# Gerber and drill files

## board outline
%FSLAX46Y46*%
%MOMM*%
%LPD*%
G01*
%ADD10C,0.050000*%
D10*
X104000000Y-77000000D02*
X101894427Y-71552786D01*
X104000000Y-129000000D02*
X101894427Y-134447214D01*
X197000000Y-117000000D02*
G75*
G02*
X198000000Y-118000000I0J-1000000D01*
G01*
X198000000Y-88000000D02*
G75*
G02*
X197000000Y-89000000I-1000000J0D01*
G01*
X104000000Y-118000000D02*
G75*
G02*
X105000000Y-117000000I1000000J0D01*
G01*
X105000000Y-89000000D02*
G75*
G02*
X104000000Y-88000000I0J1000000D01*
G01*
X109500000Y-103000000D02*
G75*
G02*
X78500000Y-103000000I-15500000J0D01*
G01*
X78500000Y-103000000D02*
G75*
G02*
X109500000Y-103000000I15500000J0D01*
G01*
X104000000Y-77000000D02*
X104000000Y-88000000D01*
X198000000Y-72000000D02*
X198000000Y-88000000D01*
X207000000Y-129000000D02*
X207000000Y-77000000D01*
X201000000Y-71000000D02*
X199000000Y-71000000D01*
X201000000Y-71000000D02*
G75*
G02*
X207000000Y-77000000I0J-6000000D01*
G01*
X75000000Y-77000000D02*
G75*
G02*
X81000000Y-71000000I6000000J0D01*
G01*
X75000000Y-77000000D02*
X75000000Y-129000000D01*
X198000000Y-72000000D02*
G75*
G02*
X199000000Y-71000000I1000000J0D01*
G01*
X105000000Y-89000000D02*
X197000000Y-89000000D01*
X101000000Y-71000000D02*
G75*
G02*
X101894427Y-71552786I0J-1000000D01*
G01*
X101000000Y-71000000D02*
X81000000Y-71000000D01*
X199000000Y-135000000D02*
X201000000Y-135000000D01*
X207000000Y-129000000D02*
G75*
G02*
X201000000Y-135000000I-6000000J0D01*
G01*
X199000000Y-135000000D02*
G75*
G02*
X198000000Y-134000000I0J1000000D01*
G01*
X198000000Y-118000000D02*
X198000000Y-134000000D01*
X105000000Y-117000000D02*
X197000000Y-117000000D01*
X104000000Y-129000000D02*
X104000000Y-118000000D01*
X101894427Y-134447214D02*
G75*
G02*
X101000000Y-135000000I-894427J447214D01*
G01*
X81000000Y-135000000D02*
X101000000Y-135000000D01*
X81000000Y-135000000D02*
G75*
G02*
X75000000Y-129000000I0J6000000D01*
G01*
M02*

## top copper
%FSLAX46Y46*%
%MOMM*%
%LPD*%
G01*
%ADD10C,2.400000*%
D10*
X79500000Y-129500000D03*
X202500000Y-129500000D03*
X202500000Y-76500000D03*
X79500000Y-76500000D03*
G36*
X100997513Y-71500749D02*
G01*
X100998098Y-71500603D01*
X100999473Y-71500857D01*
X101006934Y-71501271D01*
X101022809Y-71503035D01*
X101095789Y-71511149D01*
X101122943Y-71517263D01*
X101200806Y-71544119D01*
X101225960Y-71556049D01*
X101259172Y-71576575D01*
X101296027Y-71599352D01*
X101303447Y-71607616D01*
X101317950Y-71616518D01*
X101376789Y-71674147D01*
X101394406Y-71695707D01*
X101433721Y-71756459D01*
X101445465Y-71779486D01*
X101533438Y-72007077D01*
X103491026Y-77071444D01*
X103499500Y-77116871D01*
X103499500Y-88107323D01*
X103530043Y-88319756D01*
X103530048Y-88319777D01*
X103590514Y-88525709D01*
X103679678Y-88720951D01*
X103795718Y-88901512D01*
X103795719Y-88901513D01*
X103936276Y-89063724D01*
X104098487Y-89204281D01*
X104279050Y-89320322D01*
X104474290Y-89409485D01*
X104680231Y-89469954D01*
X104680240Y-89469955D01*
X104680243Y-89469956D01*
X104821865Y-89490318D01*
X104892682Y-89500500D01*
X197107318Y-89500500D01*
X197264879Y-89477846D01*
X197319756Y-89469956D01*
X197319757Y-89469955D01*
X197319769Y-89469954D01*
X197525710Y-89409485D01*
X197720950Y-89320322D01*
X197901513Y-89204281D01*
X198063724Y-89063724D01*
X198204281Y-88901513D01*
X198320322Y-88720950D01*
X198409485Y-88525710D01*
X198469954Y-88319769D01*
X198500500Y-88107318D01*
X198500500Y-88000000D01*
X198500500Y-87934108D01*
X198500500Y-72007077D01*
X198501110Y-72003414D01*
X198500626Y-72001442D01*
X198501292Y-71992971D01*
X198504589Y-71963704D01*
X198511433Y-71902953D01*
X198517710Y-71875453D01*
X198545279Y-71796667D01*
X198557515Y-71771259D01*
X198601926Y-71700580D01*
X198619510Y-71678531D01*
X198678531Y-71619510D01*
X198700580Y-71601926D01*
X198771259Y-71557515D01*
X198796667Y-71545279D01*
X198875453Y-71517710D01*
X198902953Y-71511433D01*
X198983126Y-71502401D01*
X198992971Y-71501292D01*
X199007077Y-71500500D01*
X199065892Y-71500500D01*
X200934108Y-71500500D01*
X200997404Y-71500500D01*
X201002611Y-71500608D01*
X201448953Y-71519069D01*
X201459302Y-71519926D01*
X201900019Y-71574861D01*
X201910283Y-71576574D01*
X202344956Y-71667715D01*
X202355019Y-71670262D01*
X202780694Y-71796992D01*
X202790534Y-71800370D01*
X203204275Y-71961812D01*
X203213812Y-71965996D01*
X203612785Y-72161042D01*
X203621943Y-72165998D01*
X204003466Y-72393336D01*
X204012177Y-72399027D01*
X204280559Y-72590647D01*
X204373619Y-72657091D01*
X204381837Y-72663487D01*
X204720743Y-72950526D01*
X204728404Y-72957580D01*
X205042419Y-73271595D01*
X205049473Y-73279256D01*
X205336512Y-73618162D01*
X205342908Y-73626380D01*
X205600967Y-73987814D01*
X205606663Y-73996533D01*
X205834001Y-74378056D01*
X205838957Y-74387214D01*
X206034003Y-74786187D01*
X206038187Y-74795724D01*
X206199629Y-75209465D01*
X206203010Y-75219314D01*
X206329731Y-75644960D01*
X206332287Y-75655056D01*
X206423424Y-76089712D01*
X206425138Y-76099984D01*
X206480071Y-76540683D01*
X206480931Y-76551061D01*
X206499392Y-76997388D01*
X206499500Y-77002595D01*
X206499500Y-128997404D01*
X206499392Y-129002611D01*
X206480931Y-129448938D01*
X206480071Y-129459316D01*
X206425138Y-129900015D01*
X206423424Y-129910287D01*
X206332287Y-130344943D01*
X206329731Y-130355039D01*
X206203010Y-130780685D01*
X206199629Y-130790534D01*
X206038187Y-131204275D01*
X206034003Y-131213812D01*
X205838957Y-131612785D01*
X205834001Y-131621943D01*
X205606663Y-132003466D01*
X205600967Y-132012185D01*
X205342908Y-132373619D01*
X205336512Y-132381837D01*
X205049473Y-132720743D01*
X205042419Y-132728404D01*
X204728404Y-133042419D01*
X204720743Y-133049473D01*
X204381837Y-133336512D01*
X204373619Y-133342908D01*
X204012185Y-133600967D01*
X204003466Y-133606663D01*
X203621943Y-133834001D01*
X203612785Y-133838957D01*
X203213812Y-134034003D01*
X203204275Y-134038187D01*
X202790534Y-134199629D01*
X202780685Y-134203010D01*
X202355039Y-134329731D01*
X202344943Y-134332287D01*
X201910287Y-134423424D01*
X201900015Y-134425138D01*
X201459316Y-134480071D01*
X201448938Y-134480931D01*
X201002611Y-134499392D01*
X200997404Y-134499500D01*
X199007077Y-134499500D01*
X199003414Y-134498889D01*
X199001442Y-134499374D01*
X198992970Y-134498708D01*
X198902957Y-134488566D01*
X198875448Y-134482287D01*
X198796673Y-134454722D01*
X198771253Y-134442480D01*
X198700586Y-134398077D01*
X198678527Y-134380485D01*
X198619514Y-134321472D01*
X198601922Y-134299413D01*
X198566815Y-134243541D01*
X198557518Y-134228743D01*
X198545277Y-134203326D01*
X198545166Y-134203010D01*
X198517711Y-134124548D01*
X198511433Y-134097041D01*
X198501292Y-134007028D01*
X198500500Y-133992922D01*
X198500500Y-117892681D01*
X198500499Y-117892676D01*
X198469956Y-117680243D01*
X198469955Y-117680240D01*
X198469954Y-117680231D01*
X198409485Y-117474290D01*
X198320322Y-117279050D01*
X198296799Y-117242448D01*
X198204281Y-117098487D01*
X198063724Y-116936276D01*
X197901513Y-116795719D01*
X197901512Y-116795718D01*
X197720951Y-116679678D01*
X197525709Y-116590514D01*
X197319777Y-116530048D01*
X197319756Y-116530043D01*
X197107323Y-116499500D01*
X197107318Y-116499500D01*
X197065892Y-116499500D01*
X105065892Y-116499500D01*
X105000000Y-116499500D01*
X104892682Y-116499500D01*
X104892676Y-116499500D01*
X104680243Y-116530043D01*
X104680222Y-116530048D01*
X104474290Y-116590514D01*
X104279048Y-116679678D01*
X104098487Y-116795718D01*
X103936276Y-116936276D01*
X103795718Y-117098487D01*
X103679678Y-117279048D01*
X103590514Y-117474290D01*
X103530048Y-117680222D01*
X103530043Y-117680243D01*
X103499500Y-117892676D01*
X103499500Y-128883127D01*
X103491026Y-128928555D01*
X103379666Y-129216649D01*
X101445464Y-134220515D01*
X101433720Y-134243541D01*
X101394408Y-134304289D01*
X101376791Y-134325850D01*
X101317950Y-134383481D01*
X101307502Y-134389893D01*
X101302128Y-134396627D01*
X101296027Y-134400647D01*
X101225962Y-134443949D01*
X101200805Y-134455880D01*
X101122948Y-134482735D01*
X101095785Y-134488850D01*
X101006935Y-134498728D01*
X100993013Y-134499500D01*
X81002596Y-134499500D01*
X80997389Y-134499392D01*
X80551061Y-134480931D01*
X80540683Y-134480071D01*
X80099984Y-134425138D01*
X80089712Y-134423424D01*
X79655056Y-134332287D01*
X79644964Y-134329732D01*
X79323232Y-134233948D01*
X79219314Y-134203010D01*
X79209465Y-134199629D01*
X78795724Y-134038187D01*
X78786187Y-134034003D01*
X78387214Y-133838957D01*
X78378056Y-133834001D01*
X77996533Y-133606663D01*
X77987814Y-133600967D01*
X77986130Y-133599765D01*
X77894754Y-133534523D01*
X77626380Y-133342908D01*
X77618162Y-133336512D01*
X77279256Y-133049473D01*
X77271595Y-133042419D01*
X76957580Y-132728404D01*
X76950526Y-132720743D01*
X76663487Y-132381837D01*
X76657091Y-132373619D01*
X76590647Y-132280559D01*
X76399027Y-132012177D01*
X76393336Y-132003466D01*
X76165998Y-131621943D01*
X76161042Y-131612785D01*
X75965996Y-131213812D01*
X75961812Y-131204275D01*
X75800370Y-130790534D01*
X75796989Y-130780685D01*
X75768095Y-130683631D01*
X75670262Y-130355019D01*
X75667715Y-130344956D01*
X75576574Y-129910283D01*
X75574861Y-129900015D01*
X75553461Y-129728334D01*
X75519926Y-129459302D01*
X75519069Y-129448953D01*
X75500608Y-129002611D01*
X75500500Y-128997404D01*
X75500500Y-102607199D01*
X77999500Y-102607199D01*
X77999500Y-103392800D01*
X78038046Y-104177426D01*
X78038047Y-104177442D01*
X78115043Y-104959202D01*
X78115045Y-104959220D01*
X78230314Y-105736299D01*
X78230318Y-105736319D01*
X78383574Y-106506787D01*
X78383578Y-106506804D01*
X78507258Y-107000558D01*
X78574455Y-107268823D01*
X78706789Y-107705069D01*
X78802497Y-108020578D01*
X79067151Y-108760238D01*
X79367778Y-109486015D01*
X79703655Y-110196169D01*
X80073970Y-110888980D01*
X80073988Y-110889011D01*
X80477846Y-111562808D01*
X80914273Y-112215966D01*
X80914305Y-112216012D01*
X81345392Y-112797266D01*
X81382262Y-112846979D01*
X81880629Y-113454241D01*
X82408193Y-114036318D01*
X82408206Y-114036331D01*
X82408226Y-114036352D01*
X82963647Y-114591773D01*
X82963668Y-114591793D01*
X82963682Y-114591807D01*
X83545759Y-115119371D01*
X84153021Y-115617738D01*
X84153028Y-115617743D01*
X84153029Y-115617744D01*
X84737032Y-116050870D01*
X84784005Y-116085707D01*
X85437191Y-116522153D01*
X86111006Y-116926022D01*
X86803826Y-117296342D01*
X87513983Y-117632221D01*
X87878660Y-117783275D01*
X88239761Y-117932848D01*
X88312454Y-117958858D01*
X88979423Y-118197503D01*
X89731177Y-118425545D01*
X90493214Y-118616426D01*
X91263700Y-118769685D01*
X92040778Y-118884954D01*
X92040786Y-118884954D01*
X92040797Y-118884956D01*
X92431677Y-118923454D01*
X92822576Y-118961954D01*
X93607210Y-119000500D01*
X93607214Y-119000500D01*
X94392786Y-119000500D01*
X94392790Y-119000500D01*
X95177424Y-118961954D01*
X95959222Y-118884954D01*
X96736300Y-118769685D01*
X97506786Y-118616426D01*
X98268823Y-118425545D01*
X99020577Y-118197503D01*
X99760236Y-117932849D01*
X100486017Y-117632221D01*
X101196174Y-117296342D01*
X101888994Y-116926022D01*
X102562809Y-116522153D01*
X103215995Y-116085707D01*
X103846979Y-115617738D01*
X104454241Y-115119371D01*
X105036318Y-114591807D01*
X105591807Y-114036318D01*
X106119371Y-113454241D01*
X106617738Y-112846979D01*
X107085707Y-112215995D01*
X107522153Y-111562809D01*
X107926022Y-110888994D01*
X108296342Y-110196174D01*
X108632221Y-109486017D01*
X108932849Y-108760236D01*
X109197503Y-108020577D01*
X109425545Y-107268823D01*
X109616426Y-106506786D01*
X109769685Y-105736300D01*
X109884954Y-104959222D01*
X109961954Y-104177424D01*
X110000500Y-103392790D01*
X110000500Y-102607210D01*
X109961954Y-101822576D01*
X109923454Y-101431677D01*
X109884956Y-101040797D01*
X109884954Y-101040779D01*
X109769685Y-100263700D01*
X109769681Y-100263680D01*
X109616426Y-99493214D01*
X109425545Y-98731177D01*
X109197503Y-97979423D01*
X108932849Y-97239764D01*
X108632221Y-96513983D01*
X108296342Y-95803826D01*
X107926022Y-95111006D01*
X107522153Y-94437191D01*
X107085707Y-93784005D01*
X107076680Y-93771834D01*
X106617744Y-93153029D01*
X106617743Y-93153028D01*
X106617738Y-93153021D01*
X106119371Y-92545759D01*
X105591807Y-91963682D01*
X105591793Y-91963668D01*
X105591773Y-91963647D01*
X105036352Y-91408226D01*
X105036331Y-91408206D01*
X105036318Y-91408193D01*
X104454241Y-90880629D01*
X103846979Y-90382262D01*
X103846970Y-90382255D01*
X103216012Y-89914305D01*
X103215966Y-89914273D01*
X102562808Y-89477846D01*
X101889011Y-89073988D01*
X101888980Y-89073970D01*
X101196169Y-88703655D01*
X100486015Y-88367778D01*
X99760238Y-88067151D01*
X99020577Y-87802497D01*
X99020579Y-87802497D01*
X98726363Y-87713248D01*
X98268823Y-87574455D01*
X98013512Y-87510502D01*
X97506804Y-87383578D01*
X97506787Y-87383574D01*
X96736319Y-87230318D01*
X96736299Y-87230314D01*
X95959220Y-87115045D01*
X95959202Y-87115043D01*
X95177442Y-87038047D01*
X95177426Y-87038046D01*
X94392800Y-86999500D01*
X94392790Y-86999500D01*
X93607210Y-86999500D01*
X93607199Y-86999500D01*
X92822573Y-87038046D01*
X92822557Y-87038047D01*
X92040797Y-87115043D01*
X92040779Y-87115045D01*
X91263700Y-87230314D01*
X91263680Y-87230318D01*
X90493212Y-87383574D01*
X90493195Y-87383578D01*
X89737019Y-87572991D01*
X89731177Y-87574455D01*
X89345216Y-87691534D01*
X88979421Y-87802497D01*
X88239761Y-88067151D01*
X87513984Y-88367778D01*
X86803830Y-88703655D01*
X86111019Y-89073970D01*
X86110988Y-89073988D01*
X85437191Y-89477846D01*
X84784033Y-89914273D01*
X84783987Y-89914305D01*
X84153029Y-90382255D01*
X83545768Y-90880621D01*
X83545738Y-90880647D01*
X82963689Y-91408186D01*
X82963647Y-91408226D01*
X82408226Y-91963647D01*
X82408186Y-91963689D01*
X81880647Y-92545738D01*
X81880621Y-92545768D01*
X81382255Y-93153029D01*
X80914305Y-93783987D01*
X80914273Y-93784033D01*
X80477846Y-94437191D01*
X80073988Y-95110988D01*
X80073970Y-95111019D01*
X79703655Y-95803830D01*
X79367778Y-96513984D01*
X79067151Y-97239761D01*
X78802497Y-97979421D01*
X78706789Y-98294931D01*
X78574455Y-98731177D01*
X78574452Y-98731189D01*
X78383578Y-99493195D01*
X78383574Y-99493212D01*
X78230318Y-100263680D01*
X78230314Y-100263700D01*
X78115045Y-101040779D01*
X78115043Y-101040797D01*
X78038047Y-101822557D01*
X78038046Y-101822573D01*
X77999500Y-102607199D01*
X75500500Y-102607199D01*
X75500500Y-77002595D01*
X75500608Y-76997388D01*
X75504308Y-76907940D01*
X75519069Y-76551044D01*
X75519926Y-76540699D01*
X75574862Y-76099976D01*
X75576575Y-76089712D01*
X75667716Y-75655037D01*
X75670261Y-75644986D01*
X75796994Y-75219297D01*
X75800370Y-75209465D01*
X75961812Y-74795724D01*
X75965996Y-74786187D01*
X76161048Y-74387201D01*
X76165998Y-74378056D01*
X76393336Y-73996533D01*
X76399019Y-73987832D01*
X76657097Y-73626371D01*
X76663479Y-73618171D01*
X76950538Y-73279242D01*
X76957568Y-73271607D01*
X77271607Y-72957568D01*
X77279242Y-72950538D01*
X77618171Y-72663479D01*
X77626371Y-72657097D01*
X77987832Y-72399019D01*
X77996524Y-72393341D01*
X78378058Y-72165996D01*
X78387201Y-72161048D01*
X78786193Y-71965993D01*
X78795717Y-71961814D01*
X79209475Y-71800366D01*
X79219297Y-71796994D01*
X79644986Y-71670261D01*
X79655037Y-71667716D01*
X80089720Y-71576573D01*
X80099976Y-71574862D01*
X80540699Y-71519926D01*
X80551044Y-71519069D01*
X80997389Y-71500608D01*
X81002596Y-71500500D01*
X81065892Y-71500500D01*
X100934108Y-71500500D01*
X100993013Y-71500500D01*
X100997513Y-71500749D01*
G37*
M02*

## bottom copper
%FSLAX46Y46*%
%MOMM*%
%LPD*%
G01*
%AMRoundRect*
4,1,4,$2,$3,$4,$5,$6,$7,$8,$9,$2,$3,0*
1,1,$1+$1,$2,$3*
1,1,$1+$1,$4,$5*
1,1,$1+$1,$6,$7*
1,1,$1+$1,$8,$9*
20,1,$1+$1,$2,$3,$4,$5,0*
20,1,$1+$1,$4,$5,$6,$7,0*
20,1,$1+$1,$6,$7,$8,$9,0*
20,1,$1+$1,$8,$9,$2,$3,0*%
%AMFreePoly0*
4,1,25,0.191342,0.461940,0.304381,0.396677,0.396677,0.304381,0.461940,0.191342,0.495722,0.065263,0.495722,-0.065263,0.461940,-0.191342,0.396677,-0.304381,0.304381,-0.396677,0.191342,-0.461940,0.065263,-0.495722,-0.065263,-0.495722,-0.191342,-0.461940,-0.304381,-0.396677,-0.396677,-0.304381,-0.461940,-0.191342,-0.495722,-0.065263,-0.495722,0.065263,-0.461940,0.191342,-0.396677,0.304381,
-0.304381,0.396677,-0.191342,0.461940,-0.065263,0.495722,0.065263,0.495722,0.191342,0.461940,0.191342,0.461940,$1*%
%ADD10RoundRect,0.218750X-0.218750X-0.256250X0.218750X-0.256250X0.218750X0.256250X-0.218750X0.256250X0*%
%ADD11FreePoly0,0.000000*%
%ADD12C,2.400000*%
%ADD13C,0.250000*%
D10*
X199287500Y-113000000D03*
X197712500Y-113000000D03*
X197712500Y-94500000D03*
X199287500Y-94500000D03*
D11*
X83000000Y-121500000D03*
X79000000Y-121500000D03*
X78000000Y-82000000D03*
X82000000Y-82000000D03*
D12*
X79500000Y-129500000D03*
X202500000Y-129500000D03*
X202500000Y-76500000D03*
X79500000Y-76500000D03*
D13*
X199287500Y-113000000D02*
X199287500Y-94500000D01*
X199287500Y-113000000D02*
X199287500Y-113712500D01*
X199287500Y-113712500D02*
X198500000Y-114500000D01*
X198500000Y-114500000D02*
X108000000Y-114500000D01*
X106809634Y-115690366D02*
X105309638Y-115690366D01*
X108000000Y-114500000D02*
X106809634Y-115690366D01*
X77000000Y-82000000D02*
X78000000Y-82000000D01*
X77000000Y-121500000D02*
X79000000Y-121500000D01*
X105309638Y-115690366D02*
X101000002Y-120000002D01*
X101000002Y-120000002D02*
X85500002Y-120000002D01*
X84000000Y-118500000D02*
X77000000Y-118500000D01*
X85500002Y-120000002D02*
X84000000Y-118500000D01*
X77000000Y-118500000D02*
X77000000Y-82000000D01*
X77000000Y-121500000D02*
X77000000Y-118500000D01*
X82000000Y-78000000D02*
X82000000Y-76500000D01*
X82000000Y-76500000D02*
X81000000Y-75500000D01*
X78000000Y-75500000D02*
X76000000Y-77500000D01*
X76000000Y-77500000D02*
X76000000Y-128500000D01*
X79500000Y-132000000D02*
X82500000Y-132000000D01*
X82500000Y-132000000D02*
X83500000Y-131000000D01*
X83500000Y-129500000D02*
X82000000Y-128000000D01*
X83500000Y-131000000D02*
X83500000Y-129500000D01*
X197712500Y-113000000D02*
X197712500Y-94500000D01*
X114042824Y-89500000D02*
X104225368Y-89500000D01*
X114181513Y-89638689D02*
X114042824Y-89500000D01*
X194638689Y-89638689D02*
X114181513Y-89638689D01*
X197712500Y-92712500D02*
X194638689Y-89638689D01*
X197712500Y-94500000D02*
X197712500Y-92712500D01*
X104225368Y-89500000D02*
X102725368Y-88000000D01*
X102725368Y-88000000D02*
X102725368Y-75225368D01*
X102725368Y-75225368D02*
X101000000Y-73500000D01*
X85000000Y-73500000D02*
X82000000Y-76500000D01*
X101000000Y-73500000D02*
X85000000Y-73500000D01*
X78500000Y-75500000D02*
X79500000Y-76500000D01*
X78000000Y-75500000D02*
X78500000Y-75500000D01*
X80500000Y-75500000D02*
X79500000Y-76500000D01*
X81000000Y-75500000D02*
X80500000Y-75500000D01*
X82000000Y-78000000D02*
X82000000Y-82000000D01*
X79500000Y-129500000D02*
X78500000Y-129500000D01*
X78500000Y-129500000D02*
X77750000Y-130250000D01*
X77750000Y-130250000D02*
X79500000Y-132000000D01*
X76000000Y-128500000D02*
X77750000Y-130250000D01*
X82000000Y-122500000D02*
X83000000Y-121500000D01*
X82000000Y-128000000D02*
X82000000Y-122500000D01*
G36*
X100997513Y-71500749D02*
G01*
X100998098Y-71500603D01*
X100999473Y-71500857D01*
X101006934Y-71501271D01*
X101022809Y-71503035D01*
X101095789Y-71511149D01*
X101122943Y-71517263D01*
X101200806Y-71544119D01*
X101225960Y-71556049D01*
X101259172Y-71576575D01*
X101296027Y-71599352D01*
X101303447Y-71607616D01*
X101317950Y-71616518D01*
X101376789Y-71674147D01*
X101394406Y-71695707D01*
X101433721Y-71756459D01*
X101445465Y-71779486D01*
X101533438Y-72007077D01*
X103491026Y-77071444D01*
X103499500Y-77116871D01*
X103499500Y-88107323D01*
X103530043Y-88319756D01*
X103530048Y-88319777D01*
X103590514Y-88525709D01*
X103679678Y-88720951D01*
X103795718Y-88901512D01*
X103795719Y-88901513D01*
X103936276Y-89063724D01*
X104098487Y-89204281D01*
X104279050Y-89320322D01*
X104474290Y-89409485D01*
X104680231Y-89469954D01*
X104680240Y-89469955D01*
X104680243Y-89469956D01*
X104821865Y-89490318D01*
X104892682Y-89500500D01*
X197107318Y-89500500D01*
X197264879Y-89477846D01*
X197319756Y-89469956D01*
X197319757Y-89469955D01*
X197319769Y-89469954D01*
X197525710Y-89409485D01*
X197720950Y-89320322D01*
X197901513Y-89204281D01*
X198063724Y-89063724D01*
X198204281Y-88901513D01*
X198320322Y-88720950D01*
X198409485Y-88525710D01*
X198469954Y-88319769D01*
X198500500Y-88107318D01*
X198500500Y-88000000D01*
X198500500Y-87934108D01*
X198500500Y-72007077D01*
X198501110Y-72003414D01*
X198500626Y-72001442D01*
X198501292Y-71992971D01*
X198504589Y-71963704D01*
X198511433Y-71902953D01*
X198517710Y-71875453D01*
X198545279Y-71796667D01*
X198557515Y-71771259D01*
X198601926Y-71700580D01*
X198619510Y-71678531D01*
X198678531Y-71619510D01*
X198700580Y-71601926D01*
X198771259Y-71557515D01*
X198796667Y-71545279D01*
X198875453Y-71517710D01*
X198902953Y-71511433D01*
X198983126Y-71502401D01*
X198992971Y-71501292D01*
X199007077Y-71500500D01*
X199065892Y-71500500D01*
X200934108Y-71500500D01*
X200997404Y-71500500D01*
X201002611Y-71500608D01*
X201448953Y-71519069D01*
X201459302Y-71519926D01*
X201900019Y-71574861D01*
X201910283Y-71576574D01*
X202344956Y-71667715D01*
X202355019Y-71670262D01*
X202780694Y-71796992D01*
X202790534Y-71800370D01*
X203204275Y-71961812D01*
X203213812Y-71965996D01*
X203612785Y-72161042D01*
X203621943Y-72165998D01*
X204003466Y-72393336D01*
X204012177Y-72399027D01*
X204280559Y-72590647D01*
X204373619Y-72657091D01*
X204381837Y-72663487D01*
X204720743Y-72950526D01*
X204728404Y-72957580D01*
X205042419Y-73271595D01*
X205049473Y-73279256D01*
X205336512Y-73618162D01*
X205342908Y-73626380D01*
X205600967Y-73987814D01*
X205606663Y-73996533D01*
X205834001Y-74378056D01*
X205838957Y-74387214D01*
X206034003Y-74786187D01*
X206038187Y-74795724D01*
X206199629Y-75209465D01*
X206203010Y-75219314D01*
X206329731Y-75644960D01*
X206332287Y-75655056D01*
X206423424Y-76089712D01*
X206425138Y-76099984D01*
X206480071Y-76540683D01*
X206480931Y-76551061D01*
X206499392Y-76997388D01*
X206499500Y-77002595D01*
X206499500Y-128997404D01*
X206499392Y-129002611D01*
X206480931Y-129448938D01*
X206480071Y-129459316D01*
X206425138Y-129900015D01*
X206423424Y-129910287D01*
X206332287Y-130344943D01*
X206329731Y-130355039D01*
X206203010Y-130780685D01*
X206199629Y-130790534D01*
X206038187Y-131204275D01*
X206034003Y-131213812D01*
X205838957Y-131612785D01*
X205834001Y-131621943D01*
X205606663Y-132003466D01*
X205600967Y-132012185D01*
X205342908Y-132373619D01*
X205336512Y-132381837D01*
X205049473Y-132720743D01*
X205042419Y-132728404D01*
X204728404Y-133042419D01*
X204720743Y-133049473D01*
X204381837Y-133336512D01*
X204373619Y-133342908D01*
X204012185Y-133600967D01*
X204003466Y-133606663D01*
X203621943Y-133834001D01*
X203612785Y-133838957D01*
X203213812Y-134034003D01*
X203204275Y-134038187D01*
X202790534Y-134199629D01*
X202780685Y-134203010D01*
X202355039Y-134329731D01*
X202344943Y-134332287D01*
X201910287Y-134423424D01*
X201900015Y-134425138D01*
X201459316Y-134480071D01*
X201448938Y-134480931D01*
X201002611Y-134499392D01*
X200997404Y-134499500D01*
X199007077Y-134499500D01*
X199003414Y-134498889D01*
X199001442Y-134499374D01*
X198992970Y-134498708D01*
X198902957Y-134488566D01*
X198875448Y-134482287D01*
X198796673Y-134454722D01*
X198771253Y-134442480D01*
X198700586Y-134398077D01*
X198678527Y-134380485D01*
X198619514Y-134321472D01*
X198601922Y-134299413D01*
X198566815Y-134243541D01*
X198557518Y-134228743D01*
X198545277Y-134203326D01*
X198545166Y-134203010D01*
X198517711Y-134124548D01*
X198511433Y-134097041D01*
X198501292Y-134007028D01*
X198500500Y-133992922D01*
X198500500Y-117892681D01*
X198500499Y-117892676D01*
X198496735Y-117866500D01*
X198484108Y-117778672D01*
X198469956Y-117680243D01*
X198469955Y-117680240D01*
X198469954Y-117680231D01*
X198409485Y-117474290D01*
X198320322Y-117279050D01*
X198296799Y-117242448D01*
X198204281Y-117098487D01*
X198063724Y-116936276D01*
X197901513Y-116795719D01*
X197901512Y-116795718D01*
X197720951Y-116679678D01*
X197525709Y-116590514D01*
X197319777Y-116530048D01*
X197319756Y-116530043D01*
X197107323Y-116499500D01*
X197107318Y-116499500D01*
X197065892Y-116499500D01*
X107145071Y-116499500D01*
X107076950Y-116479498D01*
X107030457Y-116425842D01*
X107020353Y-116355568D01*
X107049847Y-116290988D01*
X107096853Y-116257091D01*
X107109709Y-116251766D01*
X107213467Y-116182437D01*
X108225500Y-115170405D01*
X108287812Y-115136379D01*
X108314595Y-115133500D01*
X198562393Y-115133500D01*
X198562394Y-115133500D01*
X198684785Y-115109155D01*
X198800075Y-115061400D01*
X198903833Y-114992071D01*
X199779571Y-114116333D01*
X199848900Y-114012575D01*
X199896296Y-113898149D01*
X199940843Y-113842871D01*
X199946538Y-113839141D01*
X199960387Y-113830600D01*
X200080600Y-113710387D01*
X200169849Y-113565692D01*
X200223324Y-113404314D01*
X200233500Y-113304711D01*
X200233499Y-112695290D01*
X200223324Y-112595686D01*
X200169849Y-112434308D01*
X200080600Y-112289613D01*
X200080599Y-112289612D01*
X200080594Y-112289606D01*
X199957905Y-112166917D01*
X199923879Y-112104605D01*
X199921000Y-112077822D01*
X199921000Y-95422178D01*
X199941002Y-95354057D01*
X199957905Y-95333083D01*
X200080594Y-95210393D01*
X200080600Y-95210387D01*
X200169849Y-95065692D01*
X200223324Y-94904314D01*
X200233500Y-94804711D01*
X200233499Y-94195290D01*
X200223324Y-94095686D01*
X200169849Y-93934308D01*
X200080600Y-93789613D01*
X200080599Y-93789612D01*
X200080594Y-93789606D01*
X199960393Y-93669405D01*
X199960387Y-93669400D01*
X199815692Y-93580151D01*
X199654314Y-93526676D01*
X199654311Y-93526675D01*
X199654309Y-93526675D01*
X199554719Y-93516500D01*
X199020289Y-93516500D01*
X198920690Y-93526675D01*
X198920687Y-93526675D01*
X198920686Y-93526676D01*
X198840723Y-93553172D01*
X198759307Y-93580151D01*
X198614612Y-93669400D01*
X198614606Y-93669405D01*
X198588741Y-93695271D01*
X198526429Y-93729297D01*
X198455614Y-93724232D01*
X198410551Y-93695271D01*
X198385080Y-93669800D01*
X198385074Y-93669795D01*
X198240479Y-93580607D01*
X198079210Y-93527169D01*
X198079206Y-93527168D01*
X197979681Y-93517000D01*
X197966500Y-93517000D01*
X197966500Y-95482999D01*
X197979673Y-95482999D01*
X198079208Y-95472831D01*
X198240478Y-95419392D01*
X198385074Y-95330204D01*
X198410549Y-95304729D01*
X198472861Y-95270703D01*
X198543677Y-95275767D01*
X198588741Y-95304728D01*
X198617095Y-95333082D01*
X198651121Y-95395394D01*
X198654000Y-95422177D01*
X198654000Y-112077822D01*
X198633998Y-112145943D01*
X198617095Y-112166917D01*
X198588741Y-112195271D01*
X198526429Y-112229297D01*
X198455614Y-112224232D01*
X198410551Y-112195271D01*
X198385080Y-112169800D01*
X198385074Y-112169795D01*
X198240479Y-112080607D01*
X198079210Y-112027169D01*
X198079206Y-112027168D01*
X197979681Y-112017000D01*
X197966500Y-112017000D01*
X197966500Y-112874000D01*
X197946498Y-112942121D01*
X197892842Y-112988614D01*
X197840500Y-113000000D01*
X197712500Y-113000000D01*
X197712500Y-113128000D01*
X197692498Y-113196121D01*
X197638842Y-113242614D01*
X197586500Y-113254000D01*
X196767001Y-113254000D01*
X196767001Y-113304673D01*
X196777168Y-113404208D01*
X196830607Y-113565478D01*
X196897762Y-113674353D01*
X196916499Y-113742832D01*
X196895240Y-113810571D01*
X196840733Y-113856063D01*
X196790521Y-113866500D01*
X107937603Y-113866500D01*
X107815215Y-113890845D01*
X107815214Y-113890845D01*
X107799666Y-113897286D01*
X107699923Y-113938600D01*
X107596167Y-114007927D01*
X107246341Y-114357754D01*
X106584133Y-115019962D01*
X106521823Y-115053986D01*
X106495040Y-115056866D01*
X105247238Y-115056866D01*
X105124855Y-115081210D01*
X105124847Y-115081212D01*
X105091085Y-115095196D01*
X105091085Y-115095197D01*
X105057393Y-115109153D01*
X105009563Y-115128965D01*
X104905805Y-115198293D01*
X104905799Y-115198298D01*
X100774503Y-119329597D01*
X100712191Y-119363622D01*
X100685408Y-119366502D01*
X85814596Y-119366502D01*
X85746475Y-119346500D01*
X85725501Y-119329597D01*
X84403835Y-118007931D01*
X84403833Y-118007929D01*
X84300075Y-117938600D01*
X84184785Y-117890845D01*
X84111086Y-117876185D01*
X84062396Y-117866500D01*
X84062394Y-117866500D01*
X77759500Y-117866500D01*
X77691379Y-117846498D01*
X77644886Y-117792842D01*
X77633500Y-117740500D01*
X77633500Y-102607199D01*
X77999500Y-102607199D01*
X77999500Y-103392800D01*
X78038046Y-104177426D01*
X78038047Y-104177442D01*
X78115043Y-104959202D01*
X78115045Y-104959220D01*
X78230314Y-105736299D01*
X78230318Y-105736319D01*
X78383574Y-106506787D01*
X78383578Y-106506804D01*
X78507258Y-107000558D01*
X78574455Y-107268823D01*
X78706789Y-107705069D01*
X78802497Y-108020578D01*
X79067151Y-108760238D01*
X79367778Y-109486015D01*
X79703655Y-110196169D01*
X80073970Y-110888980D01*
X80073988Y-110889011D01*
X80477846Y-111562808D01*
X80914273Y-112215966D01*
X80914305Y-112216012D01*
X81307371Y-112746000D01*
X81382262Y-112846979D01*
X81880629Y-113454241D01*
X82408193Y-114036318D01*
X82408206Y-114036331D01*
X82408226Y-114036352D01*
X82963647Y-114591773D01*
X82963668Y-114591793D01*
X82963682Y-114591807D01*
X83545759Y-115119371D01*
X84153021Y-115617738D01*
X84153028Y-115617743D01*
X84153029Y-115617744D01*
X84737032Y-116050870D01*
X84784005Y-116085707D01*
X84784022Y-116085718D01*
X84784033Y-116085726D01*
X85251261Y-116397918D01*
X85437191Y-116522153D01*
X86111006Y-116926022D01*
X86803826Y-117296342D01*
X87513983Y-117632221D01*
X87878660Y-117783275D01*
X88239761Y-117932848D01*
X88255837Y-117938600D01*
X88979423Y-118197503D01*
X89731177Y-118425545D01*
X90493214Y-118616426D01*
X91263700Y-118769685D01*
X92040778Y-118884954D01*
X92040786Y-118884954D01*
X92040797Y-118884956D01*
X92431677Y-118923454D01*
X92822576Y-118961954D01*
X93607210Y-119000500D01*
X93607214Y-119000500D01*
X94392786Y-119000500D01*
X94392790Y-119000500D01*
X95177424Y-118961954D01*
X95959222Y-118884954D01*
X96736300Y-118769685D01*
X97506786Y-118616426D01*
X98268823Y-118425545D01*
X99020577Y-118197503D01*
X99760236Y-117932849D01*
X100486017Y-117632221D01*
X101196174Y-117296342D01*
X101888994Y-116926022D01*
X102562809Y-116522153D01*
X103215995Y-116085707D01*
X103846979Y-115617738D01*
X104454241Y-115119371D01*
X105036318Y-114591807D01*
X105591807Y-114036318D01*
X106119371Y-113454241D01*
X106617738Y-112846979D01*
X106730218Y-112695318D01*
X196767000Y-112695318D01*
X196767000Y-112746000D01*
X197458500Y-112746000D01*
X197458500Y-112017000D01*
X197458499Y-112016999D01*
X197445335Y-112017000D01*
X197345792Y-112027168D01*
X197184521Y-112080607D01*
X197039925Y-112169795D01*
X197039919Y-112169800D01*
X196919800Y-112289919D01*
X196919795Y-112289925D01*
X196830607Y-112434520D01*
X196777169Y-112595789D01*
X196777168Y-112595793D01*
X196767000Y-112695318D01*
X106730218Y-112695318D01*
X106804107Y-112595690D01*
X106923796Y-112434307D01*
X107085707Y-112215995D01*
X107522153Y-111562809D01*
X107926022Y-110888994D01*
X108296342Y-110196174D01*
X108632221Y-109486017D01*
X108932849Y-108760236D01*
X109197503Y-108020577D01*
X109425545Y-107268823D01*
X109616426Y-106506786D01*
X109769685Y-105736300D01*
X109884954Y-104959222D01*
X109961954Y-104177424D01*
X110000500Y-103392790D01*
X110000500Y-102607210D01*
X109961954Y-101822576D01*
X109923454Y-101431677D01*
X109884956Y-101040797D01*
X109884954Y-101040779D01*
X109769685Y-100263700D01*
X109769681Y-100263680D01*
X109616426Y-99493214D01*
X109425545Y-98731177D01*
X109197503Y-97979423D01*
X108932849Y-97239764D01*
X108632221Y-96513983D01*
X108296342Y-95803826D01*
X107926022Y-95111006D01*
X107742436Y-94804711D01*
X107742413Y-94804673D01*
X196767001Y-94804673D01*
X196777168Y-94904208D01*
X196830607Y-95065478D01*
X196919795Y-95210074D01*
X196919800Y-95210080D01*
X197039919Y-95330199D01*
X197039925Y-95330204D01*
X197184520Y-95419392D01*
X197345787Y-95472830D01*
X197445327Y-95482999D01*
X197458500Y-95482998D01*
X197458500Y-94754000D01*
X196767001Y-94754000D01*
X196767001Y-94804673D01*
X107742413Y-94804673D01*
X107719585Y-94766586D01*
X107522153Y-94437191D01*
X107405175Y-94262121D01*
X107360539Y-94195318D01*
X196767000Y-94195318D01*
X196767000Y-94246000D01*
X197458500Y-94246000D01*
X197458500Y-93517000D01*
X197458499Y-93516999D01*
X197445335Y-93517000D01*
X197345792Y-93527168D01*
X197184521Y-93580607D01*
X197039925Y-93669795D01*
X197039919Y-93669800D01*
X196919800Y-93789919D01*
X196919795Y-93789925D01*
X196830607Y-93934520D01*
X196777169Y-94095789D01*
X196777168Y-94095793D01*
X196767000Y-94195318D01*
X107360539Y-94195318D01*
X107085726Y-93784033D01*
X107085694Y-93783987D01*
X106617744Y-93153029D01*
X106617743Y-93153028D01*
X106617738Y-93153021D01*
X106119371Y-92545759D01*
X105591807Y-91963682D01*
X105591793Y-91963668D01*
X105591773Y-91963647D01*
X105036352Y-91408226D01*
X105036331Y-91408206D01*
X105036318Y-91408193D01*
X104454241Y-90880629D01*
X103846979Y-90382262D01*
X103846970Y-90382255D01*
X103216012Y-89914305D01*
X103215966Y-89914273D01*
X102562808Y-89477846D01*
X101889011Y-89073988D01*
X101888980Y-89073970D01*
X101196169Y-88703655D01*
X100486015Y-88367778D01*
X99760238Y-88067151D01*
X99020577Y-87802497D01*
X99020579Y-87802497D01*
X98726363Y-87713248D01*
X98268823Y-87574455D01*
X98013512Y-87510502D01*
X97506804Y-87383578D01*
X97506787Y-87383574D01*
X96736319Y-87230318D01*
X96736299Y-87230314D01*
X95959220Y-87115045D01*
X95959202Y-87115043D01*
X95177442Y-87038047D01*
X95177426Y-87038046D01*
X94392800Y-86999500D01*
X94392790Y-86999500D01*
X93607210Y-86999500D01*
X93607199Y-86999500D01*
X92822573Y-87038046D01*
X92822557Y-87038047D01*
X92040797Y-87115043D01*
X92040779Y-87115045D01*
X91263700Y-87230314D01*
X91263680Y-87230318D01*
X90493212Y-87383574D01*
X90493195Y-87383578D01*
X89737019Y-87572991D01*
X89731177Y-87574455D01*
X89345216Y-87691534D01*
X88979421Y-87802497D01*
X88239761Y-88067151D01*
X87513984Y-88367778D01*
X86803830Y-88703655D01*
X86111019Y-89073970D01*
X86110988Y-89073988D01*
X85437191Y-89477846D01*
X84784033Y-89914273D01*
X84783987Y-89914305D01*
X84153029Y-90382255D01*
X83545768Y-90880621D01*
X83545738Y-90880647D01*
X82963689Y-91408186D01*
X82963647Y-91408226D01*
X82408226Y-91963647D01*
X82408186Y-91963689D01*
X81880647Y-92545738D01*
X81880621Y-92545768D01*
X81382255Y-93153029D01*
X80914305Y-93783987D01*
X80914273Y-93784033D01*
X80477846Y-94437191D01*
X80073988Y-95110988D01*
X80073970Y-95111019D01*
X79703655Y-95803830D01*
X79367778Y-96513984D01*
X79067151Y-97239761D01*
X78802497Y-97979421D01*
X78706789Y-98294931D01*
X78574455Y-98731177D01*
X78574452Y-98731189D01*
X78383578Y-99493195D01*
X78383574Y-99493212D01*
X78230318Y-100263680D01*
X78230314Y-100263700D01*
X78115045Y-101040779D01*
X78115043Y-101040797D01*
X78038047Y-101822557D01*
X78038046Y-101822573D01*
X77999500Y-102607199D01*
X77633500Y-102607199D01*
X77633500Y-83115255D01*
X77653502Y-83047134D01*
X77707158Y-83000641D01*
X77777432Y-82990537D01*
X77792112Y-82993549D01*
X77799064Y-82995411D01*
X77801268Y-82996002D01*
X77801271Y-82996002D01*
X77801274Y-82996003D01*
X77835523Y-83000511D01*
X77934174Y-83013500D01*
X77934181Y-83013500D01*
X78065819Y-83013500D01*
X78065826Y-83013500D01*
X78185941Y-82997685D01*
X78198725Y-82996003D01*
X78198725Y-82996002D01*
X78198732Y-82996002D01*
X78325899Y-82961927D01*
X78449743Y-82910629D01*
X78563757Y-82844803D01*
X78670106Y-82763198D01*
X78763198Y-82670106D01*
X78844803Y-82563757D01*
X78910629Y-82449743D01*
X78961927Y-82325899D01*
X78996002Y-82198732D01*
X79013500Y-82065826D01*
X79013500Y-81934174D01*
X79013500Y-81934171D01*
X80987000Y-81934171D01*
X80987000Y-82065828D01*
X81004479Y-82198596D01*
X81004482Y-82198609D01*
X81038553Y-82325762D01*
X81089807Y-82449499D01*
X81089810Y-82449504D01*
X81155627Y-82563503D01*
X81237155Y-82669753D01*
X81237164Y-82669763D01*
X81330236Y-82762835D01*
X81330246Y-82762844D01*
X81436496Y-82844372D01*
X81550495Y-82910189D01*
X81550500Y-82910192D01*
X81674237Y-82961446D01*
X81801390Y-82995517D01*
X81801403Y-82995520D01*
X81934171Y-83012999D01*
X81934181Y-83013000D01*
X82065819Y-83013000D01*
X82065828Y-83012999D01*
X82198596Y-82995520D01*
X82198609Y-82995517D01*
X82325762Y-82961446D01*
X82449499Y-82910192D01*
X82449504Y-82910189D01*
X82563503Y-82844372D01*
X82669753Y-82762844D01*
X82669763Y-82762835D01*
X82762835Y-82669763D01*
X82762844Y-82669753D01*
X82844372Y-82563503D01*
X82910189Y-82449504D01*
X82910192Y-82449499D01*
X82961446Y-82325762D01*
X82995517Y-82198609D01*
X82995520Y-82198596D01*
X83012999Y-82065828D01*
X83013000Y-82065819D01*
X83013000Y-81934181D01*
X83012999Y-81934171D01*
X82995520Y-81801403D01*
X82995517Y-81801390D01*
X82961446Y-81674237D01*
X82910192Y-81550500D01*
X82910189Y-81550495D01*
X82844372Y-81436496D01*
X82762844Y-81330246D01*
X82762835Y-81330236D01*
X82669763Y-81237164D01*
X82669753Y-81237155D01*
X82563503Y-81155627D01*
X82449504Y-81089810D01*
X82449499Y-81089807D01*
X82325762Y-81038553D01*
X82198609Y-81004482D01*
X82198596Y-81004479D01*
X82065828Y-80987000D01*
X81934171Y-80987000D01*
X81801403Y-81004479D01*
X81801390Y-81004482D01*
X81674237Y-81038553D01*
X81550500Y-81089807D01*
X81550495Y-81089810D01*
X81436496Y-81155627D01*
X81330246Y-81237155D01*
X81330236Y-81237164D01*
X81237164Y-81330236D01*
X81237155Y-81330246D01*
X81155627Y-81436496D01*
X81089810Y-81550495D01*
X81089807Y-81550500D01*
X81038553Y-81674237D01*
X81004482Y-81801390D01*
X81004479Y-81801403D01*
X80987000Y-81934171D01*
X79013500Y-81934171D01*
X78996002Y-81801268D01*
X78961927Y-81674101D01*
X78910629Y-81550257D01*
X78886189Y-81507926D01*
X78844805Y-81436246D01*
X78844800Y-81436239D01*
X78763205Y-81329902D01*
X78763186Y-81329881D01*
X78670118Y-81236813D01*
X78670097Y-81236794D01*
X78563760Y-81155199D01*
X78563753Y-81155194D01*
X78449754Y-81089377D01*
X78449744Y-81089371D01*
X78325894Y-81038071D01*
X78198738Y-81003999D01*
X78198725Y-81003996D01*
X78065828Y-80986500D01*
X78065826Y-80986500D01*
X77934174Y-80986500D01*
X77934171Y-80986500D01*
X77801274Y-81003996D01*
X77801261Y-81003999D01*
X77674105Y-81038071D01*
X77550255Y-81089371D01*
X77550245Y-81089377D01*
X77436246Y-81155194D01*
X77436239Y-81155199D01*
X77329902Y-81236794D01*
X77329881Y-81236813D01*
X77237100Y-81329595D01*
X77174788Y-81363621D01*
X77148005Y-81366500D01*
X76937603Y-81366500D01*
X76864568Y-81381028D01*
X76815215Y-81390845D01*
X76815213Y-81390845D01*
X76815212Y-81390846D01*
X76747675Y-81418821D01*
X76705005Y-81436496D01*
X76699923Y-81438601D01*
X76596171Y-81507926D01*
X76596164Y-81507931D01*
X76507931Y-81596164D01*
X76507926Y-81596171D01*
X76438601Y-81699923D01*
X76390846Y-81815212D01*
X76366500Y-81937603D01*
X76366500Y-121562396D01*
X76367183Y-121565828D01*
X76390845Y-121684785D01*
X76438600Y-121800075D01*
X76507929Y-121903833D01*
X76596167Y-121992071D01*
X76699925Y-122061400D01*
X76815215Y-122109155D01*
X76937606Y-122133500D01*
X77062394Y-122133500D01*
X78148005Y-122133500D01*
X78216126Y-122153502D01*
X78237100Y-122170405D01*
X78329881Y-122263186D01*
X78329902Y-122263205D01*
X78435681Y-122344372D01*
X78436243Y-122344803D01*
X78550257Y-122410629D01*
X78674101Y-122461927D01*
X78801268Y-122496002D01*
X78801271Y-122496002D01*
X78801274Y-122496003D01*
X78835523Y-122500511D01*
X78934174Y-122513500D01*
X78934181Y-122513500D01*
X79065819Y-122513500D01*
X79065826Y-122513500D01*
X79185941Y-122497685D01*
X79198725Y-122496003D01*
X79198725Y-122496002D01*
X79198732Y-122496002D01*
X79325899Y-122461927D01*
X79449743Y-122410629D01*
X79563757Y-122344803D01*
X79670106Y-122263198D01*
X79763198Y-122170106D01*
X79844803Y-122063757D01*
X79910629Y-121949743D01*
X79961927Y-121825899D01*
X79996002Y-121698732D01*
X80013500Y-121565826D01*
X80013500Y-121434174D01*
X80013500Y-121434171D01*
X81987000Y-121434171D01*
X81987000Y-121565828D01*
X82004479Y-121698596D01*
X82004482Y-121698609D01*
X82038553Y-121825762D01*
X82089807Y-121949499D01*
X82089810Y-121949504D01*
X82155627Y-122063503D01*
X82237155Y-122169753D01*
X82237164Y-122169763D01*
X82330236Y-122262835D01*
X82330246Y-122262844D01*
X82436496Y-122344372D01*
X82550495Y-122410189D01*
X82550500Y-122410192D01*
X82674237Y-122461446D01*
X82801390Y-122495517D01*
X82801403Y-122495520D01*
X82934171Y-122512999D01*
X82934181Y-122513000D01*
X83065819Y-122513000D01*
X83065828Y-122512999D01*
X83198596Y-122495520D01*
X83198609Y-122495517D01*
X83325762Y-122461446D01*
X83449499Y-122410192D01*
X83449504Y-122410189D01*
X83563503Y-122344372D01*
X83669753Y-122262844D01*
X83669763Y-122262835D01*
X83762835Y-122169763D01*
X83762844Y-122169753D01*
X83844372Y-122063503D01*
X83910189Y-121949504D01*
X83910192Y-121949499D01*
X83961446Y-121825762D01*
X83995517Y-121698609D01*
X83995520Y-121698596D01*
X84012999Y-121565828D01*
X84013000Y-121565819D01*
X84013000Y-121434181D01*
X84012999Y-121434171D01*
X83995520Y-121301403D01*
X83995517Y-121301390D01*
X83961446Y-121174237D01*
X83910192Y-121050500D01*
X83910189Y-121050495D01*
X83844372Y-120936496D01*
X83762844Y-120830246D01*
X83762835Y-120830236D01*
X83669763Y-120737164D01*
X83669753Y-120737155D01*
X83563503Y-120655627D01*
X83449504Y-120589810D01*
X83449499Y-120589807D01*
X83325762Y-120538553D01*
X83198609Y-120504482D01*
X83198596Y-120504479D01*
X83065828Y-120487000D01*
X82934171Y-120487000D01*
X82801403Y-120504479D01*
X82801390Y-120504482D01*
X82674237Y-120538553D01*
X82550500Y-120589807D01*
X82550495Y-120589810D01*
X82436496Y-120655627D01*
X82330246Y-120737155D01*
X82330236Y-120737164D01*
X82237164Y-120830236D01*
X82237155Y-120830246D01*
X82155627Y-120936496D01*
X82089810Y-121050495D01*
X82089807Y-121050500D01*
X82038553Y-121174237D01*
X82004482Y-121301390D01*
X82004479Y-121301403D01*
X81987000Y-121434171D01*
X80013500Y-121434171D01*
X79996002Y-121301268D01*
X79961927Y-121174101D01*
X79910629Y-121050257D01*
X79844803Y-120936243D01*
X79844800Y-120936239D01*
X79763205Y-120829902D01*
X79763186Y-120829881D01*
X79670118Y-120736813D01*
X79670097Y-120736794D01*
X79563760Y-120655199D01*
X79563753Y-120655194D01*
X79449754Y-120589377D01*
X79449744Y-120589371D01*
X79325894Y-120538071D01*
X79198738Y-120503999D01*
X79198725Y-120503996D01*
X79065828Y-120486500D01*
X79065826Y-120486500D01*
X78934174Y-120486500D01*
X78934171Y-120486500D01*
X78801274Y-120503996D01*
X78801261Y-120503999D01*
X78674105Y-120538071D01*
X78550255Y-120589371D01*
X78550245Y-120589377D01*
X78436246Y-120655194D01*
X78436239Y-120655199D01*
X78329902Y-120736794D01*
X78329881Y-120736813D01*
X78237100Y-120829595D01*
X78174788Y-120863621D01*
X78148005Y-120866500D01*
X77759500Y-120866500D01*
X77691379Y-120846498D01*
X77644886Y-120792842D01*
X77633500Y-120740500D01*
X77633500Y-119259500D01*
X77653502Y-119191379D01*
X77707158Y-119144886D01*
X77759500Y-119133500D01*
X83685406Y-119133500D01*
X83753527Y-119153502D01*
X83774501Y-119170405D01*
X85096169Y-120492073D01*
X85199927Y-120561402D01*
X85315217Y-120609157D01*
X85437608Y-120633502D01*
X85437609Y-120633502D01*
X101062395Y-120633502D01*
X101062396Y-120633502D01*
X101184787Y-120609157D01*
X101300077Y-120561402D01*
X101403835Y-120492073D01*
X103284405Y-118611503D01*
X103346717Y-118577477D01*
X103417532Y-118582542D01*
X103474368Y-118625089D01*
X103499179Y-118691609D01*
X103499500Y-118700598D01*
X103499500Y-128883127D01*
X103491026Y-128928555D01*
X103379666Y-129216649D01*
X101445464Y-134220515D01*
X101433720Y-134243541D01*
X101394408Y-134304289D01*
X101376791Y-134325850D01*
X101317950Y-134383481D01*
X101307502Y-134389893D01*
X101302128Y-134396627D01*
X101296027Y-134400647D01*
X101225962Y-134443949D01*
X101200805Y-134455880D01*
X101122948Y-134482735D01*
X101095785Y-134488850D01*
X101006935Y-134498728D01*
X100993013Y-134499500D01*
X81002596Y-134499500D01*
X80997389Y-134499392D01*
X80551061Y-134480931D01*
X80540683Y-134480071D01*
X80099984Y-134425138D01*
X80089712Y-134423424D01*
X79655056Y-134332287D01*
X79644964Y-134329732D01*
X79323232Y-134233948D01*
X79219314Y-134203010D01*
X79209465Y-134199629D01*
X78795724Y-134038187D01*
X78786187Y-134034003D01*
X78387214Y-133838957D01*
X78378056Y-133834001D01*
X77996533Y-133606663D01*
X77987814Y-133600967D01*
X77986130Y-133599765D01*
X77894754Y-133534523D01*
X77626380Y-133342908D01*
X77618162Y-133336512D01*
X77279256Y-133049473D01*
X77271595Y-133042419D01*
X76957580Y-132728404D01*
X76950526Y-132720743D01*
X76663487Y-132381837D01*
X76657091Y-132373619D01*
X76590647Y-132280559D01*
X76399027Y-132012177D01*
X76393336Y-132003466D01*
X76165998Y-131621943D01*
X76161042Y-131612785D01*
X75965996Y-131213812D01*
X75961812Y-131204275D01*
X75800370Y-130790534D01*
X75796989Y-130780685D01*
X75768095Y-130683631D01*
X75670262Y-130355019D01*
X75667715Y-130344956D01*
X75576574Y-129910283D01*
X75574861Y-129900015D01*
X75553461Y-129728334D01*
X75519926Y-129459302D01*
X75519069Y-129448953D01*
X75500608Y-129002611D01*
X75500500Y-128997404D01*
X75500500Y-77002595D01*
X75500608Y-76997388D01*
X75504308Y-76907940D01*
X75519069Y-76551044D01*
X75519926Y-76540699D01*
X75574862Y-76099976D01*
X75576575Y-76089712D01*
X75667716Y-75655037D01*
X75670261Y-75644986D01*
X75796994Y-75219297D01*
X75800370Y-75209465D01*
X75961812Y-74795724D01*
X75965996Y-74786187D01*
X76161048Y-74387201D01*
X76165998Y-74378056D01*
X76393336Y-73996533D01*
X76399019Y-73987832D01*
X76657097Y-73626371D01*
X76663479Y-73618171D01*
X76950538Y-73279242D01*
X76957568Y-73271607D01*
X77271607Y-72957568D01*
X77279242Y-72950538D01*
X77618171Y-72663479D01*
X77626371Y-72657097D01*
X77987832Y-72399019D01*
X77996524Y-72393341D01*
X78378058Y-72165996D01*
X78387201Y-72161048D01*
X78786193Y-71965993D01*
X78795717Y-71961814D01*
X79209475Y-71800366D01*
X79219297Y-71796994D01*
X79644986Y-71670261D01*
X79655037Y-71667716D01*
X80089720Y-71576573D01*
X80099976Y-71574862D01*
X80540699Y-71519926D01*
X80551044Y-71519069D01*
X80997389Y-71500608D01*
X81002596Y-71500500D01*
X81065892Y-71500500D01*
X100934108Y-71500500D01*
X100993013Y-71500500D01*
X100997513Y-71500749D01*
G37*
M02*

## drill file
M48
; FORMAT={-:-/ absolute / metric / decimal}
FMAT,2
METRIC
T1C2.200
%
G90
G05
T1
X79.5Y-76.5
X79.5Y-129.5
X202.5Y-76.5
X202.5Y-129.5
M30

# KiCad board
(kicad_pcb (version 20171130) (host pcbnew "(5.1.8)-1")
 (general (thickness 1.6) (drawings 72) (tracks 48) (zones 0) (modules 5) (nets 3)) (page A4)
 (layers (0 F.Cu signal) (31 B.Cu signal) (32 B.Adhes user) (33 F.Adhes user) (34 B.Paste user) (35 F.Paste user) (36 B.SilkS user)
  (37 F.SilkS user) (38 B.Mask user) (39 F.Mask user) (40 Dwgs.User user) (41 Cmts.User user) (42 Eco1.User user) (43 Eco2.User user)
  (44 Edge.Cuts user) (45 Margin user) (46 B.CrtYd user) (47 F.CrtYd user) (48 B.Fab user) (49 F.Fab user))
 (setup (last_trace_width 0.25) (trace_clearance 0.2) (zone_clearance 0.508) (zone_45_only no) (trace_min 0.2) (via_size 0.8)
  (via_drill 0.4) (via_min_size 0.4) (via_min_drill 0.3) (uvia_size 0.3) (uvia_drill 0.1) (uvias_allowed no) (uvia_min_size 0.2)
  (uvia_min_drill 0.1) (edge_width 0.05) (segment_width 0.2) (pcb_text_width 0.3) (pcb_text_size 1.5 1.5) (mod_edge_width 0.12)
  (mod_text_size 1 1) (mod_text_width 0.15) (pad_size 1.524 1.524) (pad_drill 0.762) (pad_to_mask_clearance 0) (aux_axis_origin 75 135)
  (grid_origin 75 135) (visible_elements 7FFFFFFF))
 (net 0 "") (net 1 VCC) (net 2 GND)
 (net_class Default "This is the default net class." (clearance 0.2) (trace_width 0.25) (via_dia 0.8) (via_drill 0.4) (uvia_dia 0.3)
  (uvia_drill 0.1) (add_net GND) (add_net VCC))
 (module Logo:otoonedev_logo (layer F.Cu) (at 169 103 180)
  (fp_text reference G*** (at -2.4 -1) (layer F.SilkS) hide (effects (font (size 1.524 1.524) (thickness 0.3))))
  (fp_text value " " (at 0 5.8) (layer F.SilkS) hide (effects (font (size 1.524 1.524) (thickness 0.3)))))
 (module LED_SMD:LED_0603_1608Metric (layer B.Cu) (at 198.5 113)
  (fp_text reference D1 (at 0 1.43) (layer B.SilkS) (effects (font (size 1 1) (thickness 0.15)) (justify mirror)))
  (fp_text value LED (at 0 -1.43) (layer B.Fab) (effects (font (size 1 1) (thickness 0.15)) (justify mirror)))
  (pad 2 smd roundrect (at 0.7875 0) (size 0.875 0.95) (layers B.Cu B.Paste B.Mask) (roundrect_rratio 0.25) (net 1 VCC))
  (pad 1 smd roundrect (at -0.7875 0) (size 0.875 0.95) (layers B.Cu B.Paste B.Mask) (roundrect_rratio 0.25) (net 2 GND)))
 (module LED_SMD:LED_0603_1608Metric (layer B.Cu) (at 198.5 94.5)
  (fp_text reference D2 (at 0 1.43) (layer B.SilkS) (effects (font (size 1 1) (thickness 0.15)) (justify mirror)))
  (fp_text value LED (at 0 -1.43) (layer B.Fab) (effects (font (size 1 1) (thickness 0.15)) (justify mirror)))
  (pad 1 smd roundrect (at -0.7875 0) (size 0.875 0.95) (layers B.Cu B.Paste B.Mask) (roundrect_rratio 0.25) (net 2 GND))
  (pad 2 smd roundrect (at 0.7875 0) (size 0.875 0.95) (layers B.Cu B.Paste B.Mask) (roundrect_rratio 0.25) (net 1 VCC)))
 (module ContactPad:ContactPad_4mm (layer B.Cu) (at 81 121.5)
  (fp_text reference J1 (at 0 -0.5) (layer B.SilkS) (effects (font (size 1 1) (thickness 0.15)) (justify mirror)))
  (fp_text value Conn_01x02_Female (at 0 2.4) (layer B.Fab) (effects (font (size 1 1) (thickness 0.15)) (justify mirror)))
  (pad 2 smd custom (at 2 0) (size 1 1) (layers B.Cu B.Mask) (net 2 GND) (zone_connect 0) (options (clearance outline) (anchor circle))
   (primitives))
  (pad 1 smd custom (at -2 0) (size 1 1) (layers B.Cu B.Mask) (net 1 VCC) (zone_connect 0) (options (clearance outline) (anchor circle))
   (primitives)))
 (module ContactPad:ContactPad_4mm (layer B.Cu) (at 80 82)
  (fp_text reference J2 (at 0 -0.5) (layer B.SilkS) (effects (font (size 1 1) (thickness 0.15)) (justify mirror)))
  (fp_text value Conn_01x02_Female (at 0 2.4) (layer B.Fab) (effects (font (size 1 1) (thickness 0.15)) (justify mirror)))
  (pad 1 smd custom (at -2 0) (size 1 1) (layers B.Cu B.Mask) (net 1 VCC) (zone_connect 0) (options (clearance outline) (anchor circle))
   (primitives))
  (pad 2 smd custom (at 2 0) (size 1 1) (layers B.Cu B.Mask) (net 2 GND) (zone_connect 0) (options (clearance outline) (anchor circle))
   (primitives)))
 (gr_line (start 104 77) (end 101.894427 71.552786) (layer Edge.Cuts) (width 0.05))
 (gr_line (start 104 129) (end 101.894427 134.447214) (layer Edge.Cuts) (width 0.05))
 (gr_arc (start 197 118) (end 198 118) (angle -90) (layer Edge.Cuts) (width 0.05))
 (gr_arc (start 197 88) (end 197 89) (angle -90) (layer Edge.Cuts) (width 0.05))
 (gr_arc (start 105 118) (end 105 117) (angle -90) (layer Edge.Cuts) (width 0.05))
 (gr_arc (start 105 88) (end 104 88) (angle -90) (layer Edge.Cuts) (width 0.05))
 (gr_circle (center 94 103) (end 109.5 103) (layer Edge.Cuts) (width 0.05))
 (gr_line (start 104 77) (end 104 88) (layer Edge.Cuts) (width 0.05))
 (gr_line (start 198 72) (end 198 88) (layer Edge.Cuts) (width 0.05))
 (gr_line (start 207 129) (end 207 77) (layer Edge.Cuts) (width 0.05))
 (gr_line (start 201 71) (end 199 71) (layer Edge.Cuts) (width 0.05))
 (gr_arc (start 201 77) (end 207 77) (angle -90) (layer Edge.Cuts) (width 0.05))
 (gr_arc (start 81 77) (end 81 71) (angle -90) (layer Edge.Cuts) (width 0.05))
 (gr_line (start 75 77) (end 75 129) (layer Edge.Cuts) (width 0.05))
 (gr_arc (start 199 72) (end 199 71) (angle -90) (layer Edge.Cuts) (width 0.05))
 (gr_line (start 105 89) (end 197 89) (layer Edge.Cuts) (width 0.05))
 (gr_arc (start 101 72) (end 101 71) (angle 63.43494882) (layer Edge.Cuts) (width 0.05))
 (gr_line (start 101 71) (end 81 71) (layer Edge.Cuts) (width 0.05))
 (gr_line (start 199 135) (end 201 135) (layer Edge.Cuts) (width 0.05))
 (gr_arc (start 201 129) (end 201 135) (angle -90) (layer Edge.Cuts) (width 0.05))
 (gr_arc (start 199 134) (end 198 134) (angle -90) (layer Edge.Cuts) (width 0.05))
 (gr_line (start 198 118) (end 198 134) (layer Edge.Cuts) (width 0.05))
 (gr_line (start 105 117) (end 197 117) (layer Edge.Cuts) (width 0.05))
 (gr_line (start 104 129) (end 104 118) (layer Edge.Cuts) (width 0.05))
 (gr_arc (start 101 134) (end 101 135) (angle -63.43494882) (layer Edge.Cuts) (width 0.05))
 (gr_line (start 81 135) (end 101 135) (layer Edge.Cuts) (width 0.05))
 (gr_arc (start 81 129) (end 75 129) (angle -90) (layer Edge.Cuts) (width 0.05))
 (segment (start 199.2875 113) (end 199.2875 94.5) (width 0.25) (layer B.Cu) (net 1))
 (segment (start 199.2875 113) (end 199.2875 113.7125) (width 0.25) (layer B.Cu) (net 1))
 (segment (start 199.2875 113.7125) (end 198.5 114.5) (width 0.25) (layer B.Cu) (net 1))
 (segment (start 198.5 114.5) (end 108 114.5) (width 0.25) (layer B.Cu) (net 1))
 (segment (start 106.809634 115.690366) (end 105.309638 115.690366) (width 0.25) (layer B.Cu) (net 1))
 (segment (start 108 114.5) (end 106.809634 115.690366) (width 0.25) (layer B.Cu) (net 1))
 (segment (start 77 82) (end 78 82) (width 0.25) (layer B.Cu) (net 1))
 (segment (start 77 121.5) (end 79 121.5) (width 0.25) (layer B.Cu) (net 1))
 (segment (start 105.309638 115.690366) (end 101.000002 120.000002) (width 0.25) (layer B.Cu) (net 1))
 (segment (start 101.000002 120.000002) (end 85.500002 120.000002) (width 0.25) (layer B.Cu) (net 1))
 (segment (start 84 118.5) (end 77 118.5) (width 0.25) (layer B.Cu) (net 1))
 (segment (start 85.500002 120.000002) (end 84 118.5) (width 0.25) (layer B.Cu) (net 1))
 (segment (start 77 118.5) (end 77 82) (width 0.25) (layer B.Cu) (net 1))
 (segment (start 77 121.5) (end 77 118.5) (width 0.25) (layer B.Cu) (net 1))
 (via (at 79.5 129.5) (size 2.4) (drill 2.2) (layers F.Cu B.Cu) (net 2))
 (via (at 202.5 129.5) (size 2.4) (drill 2.2) (layers F.Cu B.Cu) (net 2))
 (via (at 202.5 76.5) (size 2.4) (drill 2.2) (layers F.Cu B.Cu) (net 2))
 (via (at 79.5 76.5) (size 2.4) (drill 2.2) (layers F.Cu B.Cu) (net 2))
 (segment (start 82 78) (end 82 76.5) (width 0.25) (layer B.Cu) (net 2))
 (segment (start 82 76.5) (end 81 75.5) (width 0.25) (layer B.Cu) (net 2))
 (segment (start 78 75.5) (end 76 77.5) (width 0.25) (layer B.Cu) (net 2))
 (segment (start 76 77.5) (end 76 128.5) (width 0.25) (layer B.Cu) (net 2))
 (segment (start 79.5 132) (end 82.5 132) (width 0.25) (layer B.Cu) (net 2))
 (segment (start 82.5 132) (end 83.5 131) (width 0.25) (layer B.Cu) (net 2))
 (segment (start 83.5 129.5) (end 82 128) (width 0.25) (layer B.Cu) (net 2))
 (segment (start 83.5 131) (end 83.5 129.5) (width 0.25) (layer B.Cu) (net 2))
 (segment (start 197.7125 113) (end 197.7125 94.5) (width 0.25) (layer B.Cu) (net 2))
 (segment (start 114.042824 89.5) (end 104.225368 89.5) (width 0.25) (layer B.Cu) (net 2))
 (segment (start 114.181513 89.638689) (end 114.042824 89.5) (width 0.25) (layer B.Cu) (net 2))
 (segment (start 194.638689 89.638689) (end 114.181513 89.638689) (width 0.25) (layer B.Cu) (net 2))
 (segment (start 197.7125 92.7125) (end 194.638689 89.638689) (width 0.25) (layer B.Cu) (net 2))
 (segment (start 197.7125 94.5) (end 197.7125 92.7125) (width 0.25) (layer B.Cu) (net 2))
 (segment (start 104.225368 89.5) (end 102.725368 88) (width 0.25) (layer B.Cu) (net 2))
 (segment (start 102.725368 88) (end 102.725368 75.225368) (width 0.25) (layer B.Cu) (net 2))
 (segment (start 102.725368 75.225368) (end 101 73.5) (width 0.25) (layer B.Cu) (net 2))
 (segment (start 85 73.5) (end 82 76.5) (width 0.25) (layer B.Cu) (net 2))
 (segment (start 101 73.5) (end 85 73.5) (width 0.25) (layer B.Cu) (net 2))
 (segment (start 78.5 75.5) (end 79.5 76.5) (width 0.25) (layer B.Cu) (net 2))
 (segment (start 78 75.5) (end 78.5 75.5) (width 0.25) (layer B.Cu) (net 2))
 (segment (start 80.5 75.5) (end 79.5 76.5) (width 0.25) (layer B.Cu) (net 2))
 (segment (start 81 75.5) (end 80.5 75.5) (width 0.25) (layer B.Cu) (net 2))
 (segment (start 82 78) (end 82 82) (width 0.25) (layer B.Cu) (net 2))
 (segment (start 79.5 129.5) (end 78.5 129.5) (width 0.25) (layer B.Cu) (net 2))
 (segment (start 78.5 129.5) (end 77.75 130.25) (width 0.25) (layer B.Cu) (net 2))
 (segment (start 77.75 130.25) (end 79.5 132) (width 0.25) (layer B.Cu) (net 2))
 (segment (start 76 128.5) (end 77.75 130.25) (width 0.25) (layer B.Cu) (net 2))
 (segment (start 82 122.5) (end 83 121.5) (width 0.25) (layer B.Cu) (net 2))
 (segment (start 82 128) (end 82 122.5) (width 0.25) (layer B.Cu) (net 2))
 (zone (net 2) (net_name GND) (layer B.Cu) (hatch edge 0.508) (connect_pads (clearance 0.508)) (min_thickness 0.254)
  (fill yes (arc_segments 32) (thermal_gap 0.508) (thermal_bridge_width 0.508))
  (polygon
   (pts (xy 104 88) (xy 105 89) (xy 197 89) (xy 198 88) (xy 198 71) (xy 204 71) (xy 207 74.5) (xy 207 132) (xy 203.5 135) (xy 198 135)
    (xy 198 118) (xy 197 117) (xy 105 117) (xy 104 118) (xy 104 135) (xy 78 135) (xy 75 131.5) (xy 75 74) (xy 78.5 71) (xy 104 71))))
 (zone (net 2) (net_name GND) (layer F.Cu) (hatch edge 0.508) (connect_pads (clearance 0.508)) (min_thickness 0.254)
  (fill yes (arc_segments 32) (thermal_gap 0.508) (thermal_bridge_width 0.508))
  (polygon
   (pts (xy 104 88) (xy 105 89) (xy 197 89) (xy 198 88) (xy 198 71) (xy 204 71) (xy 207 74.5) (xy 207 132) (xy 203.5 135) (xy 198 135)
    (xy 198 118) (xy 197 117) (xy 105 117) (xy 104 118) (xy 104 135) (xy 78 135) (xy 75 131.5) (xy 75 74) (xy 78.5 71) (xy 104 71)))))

